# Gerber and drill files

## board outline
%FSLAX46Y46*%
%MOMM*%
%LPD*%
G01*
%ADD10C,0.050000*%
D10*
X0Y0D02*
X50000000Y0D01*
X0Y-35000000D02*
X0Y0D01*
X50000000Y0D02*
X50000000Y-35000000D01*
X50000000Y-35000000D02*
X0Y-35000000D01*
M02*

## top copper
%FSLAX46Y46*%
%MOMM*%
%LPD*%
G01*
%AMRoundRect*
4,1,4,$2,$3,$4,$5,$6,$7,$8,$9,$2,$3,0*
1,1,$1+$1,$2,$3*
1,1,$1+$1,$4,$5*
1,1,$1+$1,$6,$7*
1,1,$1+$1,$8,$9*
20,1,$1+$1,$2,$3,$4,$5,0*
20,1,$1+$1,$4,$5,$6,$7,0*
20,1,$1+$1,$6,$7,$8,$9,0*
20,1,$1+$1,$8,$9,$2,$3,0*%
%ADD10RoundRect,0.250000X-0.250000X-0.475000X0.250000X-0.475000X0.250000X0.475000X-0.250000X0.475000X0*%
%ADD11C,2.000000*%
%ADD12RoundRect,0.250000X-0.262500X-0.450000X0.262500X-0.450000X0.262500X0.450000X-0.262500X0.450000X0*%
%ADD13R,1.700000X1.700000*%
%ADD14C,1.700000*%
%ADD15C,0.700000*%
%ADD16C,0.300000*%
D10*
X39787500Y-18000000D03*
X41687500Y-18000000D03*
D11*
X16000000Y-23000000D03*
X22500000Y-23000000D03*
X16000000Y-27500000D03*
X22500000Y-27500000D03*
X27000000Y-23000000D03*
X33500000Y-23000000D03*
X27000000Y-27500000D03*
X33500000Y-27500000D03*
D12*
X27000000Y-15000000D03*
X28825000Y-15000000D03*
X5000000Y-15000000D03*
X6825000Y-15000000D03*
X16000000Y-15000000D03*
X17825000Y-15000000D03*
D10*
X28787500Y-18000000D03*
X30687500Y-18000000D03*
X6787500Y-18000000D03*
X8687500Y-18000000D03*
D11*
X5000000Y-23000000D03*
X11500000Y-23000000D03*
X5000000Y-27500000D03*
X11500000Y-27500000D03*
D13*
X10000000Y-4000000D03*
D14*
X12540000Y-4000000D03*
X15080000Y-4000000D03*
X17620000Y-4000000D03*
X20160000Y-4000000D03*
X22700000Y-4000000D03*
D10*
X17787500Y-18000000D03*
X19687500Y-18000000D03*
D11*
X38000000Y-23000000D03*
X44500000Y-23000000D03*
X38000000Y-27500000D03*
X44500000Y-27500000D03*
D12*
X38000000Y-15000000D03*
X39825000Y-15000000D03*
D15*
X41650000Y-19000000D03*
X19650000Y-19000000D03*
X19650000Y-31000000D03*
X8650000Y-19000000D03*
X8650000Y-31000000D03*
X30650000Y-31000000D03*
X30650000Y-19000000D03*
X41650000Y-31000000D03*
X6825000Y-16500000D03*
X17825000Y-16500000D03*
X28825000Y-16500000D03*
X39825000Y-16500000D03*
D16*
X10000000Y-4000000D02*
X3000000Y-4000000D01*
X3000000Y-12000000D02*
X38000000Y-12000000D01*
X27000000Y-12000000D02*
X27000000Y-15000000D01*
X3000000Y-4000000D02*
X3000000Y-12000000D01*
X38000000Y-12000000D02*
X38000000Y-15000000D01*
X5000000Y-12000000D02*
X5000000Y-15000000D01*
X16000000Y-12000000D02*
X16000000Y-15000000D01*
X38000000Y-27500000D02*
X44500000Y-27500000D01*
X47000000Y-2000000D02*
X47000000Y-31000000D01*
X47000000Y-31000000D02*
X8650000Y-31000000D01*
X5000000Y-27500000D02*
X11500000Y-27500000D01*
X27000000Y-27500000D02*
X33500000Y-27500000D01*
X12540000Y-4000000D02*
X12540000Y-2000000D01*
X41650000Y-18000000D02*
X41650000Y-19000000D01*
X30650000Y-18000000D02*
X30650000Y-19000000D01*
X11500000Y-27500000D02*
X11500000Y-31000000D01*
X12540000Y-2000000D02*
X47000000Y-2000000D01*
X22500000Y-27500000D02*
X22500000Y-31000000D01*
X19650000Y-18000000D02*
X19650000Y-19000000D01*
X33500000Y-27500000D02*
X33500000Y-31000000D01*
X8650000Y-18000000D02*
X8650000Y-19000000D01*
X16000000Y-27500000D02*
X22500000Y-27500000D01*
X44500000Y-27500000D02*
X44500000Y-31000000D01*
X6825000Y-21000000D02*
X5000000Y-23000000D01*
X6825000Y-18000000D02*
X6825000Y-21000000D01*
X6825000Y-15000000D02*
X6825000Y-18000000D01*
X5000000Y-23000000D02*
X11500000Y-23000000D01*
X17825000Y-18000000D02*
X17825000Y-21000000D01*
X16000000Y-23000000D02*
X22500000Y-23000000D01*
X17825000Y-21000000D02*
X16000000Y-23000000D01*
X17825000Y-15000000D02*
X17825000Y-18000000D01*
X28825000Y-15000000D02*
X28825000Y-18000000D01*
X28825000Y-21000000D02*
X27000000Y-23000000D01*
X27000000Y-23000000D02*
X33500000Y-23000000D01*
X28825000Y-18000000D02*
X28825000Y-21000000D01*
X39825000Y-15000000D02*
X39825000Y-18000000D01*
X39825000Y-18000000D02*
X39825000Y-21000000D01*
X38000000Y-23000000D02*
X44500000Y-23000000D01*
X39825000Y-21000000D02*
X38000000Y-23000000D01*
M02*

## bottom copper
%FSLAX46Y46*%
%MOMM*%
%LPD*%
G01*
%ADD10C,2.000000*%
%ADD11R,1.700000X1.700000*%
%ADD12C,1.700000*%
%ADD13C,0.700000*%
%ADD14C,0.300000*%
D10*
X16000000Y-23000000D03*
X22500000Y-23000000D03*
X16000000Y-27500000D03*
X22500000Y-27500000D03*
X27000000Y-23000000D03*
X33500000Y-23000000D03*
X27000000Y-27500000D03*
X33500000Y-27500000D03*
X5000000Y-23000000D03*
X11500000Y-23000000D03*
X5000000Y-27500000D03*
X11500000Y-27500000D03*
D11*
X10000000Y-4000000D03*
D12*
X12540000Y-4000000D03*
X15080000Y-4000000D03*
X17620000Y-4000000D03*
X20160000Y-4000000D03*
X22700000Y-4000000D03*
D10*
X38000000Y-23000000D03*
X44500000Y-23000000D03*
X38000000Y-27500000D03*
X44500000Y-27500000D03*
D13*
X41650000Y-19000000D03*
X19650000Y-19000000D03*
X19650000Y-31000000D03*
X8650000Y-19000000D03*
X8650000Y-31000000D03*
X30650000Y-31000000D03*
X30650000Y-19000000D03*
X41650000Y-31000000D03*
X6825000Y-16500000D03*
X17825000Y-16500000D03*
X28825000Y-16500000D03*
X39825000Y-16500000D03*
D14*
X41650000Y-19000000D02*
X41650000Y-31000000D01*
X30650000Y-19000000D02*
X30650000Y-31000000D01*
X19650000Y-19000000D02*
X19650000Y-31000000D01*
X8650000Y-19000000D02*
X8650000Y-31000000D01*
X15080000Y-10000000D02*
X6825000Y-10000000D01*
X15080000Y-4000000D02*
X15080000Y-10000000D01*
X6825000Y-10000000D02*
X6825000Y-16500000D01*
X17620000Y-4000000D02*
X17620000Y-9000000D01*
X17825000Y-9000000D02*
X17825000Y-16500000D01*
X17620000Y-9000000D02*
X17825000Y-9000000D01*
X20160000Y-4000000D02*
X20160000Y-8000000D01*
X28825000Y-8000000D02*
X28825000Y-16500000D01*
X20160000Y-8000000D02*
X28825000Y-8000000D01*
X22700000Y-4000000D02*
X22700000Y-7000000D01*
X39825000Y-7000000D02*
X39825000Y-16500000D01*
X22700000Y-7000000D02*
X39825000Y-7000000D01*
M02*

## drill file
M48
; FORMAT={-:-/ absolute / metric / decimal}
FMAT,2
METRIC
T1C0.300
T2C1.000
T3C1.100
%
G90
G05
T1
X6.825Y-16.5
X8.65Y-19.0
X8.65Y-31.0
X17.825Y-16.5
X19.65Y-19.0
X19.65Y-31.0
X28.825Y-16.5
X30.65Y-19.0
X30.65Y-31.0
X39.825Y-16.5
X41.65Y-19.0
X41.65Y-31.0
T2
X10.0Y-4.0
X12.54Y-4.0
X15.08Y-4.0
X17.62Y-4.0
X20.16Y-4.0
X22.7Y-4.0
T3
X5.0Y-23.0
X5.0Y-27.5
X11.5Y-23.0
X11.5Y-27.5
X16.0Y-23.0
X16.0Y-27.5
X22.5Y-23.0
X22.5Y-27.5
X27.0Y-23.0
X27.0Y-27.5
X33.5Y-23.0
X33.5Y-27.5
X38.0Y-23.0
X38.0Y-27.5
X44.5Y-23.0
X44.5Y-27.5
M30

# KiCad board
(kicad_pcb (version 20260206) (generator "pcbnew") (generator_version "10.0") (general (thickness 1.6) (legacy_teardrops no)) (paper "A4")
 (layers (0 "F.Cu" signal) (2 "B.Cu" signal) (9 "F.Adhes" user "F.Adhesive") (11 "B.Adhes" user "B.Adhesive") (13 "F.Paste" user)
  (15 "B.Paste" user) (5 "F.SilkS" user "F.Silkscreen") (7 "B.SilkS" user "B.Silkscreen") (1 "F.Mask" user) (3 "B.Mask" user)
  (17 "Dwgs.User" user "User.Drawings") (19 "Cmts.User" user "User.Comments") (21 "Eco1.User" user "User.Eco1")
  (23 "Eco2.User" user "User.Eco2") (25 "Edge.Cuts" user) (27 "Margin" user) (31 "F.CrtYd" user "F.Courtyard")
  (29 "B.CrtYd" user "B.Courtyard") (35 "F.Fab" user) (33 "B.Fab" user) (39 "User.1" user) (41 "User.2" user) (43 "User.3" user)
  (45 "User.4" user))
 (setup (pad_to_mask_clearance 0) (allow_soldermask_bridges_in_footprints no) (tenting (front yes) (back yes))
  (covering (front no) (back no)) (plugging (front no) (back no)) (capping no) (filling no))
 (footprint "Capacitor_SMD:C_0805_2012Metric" (layer "F.Cu") (at 40.7375 18)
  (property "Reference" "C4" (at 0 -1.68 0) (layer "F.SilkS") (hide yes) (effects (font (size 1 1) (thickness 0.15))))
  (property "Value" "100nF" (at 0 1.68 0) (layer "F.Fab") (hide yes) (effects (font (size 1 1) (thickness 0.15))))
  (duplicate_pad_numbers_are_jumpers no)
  (pad "1" smd roundrect (at -0.95 0) (size 1 1.45) (layers "F.Cu" "F.Mask" "F.Paste") (roundrect_rratio 0.25) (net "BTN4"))
  (pad "2" smd roundrect (at 0.95 0) (size 1 1.45) (layers "F.Cu" "F.Mask" "F.Paste") (roundrect_rratio 0.25) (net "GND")))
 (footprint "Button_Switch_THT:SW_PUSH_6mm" (layer "F.Cu") (at 16 23)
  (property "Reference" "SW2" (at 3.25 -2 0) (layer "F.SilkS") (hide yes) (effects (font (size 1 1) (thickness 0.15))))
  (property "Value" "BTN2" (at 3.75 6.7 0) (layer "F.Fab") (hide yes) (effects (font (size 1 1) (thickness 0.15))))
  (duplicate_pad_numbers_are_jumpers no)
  (pad "1" thru_hole circle (at 0 0 90) (size 2 2) (drill 1.1) (layers "*.Cu" "*.Mask") (remove_unused_layers no) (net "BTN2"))
  (pad "1" thru_hole circle (at 6.5 0 90) (size 2 2) (drill 1.1) (layers "*.Cu" "*.Mask") (remove_unused_layers no) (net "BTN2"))
  (pad "2" thru_hole circle (at 0 4.5 90) (size 2 2) (drill 1.1) (layers "*.Cu" "*.Mask") (remove_unused_layers no) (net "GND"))
  (pad "2" thru_hole circle (at 6.5 4.5 90) (size 2 2) (drill 1.1) (layers "*.Cu" "*.Mask") (remove_unused_layers no) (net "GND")))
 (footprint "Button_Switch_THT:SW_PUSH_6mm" (layer "F.Cu") (at 27 23)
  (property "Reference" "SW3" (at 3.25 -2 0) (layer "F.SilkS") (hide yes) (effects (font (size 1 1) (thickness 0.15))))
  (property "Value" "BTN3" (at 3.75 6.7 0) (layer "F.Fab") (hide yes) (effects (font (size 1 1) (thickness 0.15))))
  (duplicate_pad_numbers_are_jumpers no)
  (pad "1" thru_hole circle (at 0 0 90) (size 2 2) (drill 1.1) (layers "*.Cu" "*.Mask") (remove_unused_layers no) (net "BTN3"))
  (pad "1" thru_hole circle (at 6.5 0 90) (size 2 2) (drill 1.1) (layers "*.Cu" "*.Mask") (remove_unused_layers no) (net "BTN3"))
  (pad "2" thru_hole circle (at 0 4.5 90) (size 2 2) (drill 1.1) (layers "*.Cu" "*.Mask") (remove_unused_layers no) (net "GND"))
  (pad "2" thru_hole circle (at 6.5 4.5 90) (size 2 2) (drill 1.1) (layers "*.Cu" "*.Mask") (remove_unused_layers no) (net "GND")))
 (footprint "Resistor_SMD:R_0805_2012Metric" (layer "F.Cu") (at 27.9125 15)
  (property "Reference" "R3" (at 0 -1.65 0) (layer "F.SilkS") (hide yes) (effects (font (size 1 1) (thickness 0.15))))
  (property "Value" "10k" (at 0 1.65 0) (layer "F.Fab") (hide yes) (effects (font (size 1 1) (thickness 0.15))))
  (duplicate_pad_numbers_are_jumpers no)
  (pad "1" smd roundrect (at -0.9125 0) (size 1.025 1.4) (layers "F.Cu" "F.Mask" "F.Paste") (roundrect_rratio 0.243902) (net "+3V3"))
  (pad "2" smd roundrect (at 0.9125 0) (size 1.025 1.4) (layers "F.Cu" "F.Mask" "F.Paste") (roundrect_rratio 0.243902) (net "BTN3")))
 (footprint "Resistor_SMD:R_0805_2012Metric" (layer "F.Cu") (at 5.9125 15)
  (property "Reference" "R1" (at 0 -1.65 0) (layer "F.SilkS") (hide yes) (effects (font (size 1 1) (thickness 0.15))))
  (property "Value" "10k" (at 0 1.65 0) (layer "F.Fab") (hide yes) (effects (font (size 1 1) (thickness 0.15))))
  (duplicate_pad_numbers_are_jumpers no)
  (pad "1" smd roundrect (at -0.9125 0) (size 1.025 1.4) (layers "F.Cu" "F.Mask" "F.Paste") (roundrect_rratio 0.243902) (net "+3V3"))
  (pad "2" smd roundrect (at 0.9125 0) (size 1.025 1.4) (layers "F.Cu" "F.Mask" "F.Paste") (roundrect_rratio 0.243902) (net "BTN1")))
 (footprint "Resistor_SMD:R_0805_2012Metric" (layer "F.Cu") (at 16.9125 15)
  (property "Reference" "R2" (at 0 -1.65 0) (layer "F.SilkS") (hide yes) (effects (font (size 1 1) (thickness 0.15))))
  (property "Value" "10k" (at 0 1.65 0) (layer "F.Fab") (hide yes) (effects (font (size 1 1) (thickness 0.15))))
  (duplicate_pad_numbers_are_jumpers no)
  (pad "1" smd roundrect (at -0.9125 0) (size 1.025 1.4) (layers "F.Cu" "F.Mask" "F.Paste") (roundrect_rratio 0.243902) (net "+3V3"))
  (pad "2" smd roundrect (at 0.9125 0) (size 1.025 1.4) (layers "F.Cu" "F.Mask" "F.Paste") (roundrect_rratio 0.243902) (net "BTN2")))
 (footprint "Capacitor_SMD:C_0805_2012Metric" (layer "F.Cu") (at 29.7375 18)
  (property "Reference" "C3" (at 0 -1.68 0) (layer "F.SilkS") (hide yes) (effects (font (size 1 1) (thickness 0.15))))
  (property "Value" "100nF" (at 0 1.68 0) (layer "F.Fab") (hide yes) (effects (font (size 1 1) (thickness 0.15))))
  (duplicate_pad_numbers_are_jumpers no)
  (pad "1" smd roundrect (at -0.95 0) (size 1 1.45) (layers "F.Cu" "F.Mask" "F.Paste") (roundrect_rratio 0.25) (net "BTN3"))
  (pad "2" smd roundrect (at 0.95 0) (size 1 1.45) (layers "F.Cu" "F.Mask" "F.Paste") (roundrect_rratio 0.25) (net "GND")))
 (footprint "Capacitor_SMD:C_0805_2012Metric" (layer "F.Cu") (at 7.7375 18)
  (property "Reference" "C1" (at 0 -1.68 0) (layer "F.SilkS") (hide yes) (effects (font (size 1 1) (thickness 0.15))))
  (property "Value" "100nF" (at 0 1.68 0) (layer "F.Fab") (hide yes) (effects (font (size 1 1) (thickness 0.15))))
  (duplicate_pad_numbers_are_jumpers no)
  (pad "1" smd roundrect (at -0.95 0) (size 1 1.45) (layers "F.Cu" "F.Mask" "F.Paste") (roundrect_rratio 0.25) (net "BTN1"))
  (pad "2" smd roundrect (at 0.95 0) (size 1 1.45) (layers "F.Cu" "F.Mask" "F.Paste") (roundrect_rratio 0.25) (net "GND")))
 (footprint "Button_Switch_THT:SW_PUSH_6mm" (layer "F.Cu") (at 5 23)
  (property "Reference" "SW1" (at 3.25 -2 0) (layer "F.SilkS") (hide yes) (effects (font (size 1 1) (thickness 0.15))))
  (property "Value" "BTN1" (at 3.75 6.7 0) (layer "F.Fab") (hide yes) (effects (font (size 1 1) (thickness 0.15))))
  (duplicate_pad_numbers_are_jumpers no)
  (pad "1" thru_hole circle (at 0 0 90) (size 2 2) (drill 1.1) (layers "*.Cu" "*.Mask") (remove_unused_layers no) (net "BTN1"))
  (pad "1" thru_hole circle (at 6.5 0 90) (size 2 2) (drill 1.1) (layers "*.Cu" "*.Mask") (remove_unused_layers no) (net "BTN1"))
  (pad "2" thru_hole circle (at 0 4.5 90) (size 2 2) (drill 1.1) (layers "*.Cu" "*.Mask") (remove_unused_layers no) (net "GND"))
  (pad "2" thru_hole circle (at 6.5 4.5 90) (size 2 2) (drill 1.1) (layers "*.Cu" "*.Mask") (remove_unused_layers no) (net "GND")))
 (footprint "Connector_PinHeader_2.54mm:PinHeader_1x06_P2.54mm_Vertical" (layer "F.Cu") (at 10 4 90)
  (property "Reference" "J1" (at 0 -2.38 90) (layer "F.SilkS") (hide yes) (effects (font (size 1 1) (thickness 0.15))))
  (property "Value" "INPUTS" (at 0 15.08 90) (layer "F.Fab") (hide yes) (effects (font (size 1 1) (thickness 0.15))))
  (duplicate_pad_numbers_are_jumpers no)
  (pad "1" thru_hole rect (at 0 0 90) (size 1.7 1.7) (drill 1) (layers "*.Cu" "*.Mask") (remove_unused_layers no) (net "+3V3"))
  (pad "2" thru_hole circle (at 0 2.54 90) (size 1.7 1.7) (drill 1) (layers "*.Cu" "*.Mask") (remove_unused_layers no) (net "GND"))
  (pad "3" thru_hole circle (at 0 5.08 90) (size 1.7 1.7) (drill 1) (layers "*.Cu" "*.Mask") (remove_unused_layers no) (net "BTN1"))
  (pad "4" thru_hole circle (at 0 7.62 90) (size 1.7 1.7) (drill 1) (layers "*.Cu" "*.Mask") (remove_unused_layers no) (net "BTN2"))
  (pad "5" thru_hole circle (at 0 10.16 90) (size 1.7 1.7) (drill 1) (layers "*.Cu" "*.Mask") (remove_unused_layers no) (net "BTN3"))
  (pad "6" thru_hole circle (at 0 12.7 90) (size 1.7 1.7) (drill 1) (layers "*.Cu" "*.Mask") (remove_unused_layers no) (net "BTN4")))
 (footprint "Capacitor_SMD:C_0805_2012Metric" (layer "F.Cu") (at 18.7375 18)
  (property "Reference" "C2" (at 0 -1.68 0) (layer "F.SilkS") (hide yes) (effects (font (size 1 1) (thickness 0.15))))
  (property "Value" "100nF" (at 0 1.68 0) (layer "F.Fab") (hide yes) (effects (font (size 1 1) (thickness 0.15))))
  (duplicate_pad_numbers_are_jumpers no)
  (pad "1" smd roundrect (at -0.95 0) (size 1 1.45) (layers "F.Cu" "F.Mask" "F.Paste") (roundrect_rratio 0.25) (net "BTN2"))
  (pad "2" smd roundrect (at 0.95 0) (size 1 1.45) (layers "F.Cu" "F.Mask" "F.Paste") (roundrect_rratio 0.25) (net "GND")))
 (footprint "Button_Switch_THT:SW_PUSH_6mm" (layer "F.Cu") (at 38 23)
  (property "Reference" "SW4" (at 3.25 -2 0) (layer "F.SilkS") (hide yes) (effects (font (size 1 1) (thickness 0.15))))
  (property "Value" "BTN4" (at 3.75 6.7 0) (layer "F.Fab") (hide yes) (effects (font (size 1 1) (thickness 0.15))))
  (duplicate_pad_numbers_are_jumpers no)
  (pad "1" thru_hole circle (at 0 0 90) (size 2 2) (drill 1.1) (layers "*.Cu" "*.Mask") (remove_unused_layers no) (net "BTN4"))
  (pad "1" thru_hole circle (at 6.5 0 90) (size 2 2) (drill 1.1) (layers "*.Cu" "*.Mask") (remove_unused_layers no) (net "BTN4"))
  (pad "2" thru_hole circle (at 0 4.5 90) (size 2 2) (drill 1.1) (layers "*.Cu" "*.Mask") (remove_unused_layers no) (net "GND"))
  (pad "2" thru_hole circle (at 6.5 4.5 90) (size 2 2) (drill 1.1) (layers "*.Cu" "*.Mask") (remove_unused_layers no) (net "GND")))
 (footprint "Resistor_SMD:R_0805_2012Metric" (layer "F.Cu") (at 38.9125 15)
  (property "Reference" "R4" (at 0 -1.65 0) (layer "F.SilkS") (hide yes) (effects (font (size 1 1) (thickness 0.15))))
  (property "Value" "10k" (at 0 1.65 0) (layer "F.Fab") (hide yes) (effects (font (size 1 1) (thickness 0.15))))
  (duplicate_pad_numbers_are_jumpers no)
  (pad "1" smd roundrect (at -0.9125 0) (size 1.025 1.4) (layers "F.Cu" "F.Mask" "F.Paste") (roundrect_rratio 0.243902) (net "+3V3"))
  (pad "2" smd roundrect (at 0.9125 0) (size 1.025 1.4) (layers "F.Cu" "F.Mask" "F.Paste") (roundrect_rratio 0.243902) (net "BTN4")))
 (gr_line (start 0 0) (end 50 0) (stroke (width 0.05) (type default)) (layer "Edge.Cuts"))
 (gr_line (start 0 35) (end 0 0) (stroke (width 0.05) (type default)) (layer "Edge.Cuts"))
 (gr_line (start 50 0) (end 50 35) (stroke (width 0.05) (type default)) (layer "Edge.Cuts"))
 (gr_line (start 50 35) (end 0 35) (stroke (width 0.05) (type default)) (layer "Edge.Cuts"))
 (segment (start 10 4) (end 3 4) (width 0.3) (layer "F.Cu") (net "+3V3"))
 (segment (start 3 12) (end 38 12) (width 0.3) (layer "F.Cu") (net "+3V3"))
 (segment (start 27 12) (end 27 15) (width 0.3) (layer "F.Cu") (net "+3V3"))
 (segment (start 3 4) (end 3 12) (width 0.3) (layer "F.Cu") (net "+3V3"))
 (segment (start 38 12) (end 38 15) (width 0.3) (layer "F.Cu") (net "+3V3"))
 (segment (start 5 12) (end 5 15) (width 0.3) (layer "F.Cu") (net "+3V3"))
 (segment (start 16 12) (end 16 15) (width 0.3) (layer "F.Cu") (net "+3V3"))
 (segment (start 38 27.5) (end 44.5 27.5) (width 0.3) (layer "F.Cu") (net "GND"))
 (segment (start 47 2) (end 47 31) (width 0.3) (layer "F.Cu") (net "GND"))
 (segment (start 47 31) (end 8.65 31) (width 0.3) (layer "F.Cu") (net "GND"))
 (segment (start 5 27.5) (end 11.5 27.5) (width 0.3) (layer "F.Cu") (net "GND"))
 (segment (start 27 27.5) (end 33.5 27.5) (width 0.3) (layer "F.Cu") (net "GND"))
 (segment (start 12.54 4) (end 12.54 2) (width 0.3) (layer "F.Cu") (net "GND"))
 (segment (start 41.65 18) (end 41.65 19) (width 0.3) (layer "F.Cu") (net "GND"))
 (segment (start 30.65 18) (end 30.65 19) (width 0.3) (layer "F.Cu") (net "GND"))
 (segment (start 11.5 27.5) (end 11.5 31) (width 0.3) (layer "F.Cu") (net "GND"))
 (segment (start 12.54 2) (end 47 2) (width 0.3) (layer "F.Cu") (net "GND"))
 (segment (start 22.5 27.5) (end 22.5 31) (width 0.3) (layer "F.Cu") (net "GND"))
 (segment (start 19.65 18) (end 19.65 19) (width 0.3) (layer "F.Cu") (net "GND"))
 (segment (start 33.5 27.5) (end 33.5 31) (width 0.3) (layer "F.Cu") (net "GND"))
 (segment (start 8.65 18) (end 8.65 19) (width 0.3) (layer "F.Cu") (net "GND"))
 (segment (start 16 27.5) (end 22.5 27.5) (width 0.3) (layer "F.Cu") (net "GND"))
 (segment (start 44.5 27.5) (end 44.5 31) (width 0.3) (layer "F.Cu") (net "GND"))
 (via (at 41.65 19) (size 0.7) (drill 0.3) (layers "F.Cu" "B.Cu") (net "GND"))
 (via (at 19.65 19) (size 0.7) (drill 0.3) (layers "F.Cu" "B.Cu") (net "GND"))
 (via (at 19.65 31) (size 0.7) (drill 0.3) (layers "F.Cu" "B.Cu") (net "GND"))
 (via (at 8.65 19) (size 0.7) (drill 0.3) (layers "F.Cu" "B.Cu") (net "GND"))
 (via (at 8.65 31) (size 0.7) (drill 0.3) (layers "F.Cu" "B.Cu") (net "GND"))
 (via (at 30.65 31) (size 0.7) (drill 0.3) (layers "F.Cu" "B.Cu") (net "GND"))
 (via (at 30.65 19) (size 0.7) (drill 0.3) (layers "F.Cu" "B.Cu") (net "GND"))
 (via (at 41.65 31) (size 0.7) (drill 0.3) (layers "F.Cu" "B.Cu") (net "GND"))
 (segment (start 41.65 19) (end 41.65 31) (width 0.3) (layer "B.Cu") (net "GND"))
 (segment (start 30.65 19) (end 30.65 31) (width 0.3) (layer "B.Cu") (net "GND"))
 (segment (start 19.65 19) (end 19.65 31) (width 0.3) (layer "B.Cu") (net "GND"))
 (segment (start 8.65 19) (end 8.65 31) (width 0.3) (layer "B.Cu") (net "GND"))
 (segment (start 6.825 21) (end 5 23) (width 0.3) (layer "F.Cu") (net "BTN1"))
 (segment (start 6.825 18) (end 6.825 21) (width 0.3) (layer "F.Cu") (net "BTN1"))
 (segment (start 6.825 15) (end 6.825 18) (width 0.3) (layer "F.Cu") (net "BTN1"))
 (segment (start 5 23) (end 11.5 23) (width 0.3) (layer "F.Cu") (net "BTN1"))
 (via (at 6.825 16.5) (size 0.7) (drill 0.3) (layers "F.Cu" "B.Cu") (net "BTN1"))
 (segment (start 15.08 10) (end 6.825 10) (width 0.3) (layer "B.Cu") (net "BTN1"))
 (segment (start 15.08 4) (end 15.08 10) (width 0.3) (layer "B.Cu") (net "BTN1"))
 (segment (start 6.825 10) (end 6.825 16.5) (width 0.3) (layer "B.Cu") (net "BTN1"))
 (segment (start 17.825 18) (end 17.825 21) (width 0.3) (layer "F.Cu") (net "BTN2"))
 (segment (start 16 23) (end 22.5 23) (width 0.3) (layer "F.Cu") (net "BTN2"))
 (segment (start 17.825 21) (end 16 23) (width 0.3) (layer "F.Cu") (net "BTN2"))
 (segment (start 17.825 15) (end 17.825 18) (width 0.3) (layer "F.Cu") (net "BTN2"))
 (via (at 17.825 16.5) (size 0.7) (drill 0.3) (layers "F.Cu" "B.Cu") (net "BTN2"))
 (segment (start 17.62 4) (end 17.62 9) (width 0.3) (layer "B.Cu") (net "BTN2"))
 (segment (start 17.825 9) (end 17.825 16.5) (width 0.3) (layer "B.Cu") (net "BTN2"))
 (segment (start 17.62 9) (end 17.825 9) (width 0.3) (layer "B.Cu") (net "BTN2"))
 (segment (start 28.825 15) (end 28.825 18) (width 0.3) (layer "F.Cu") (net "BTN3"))
 (segment (start 28.825 21) (end 27 23) (width 0.3) (layer "F.Cu") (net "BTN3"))
 (segment (start 27 23) (end 33.5 23) (width 0.3) (layer "F.Cu") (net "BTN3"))
 (segment (start 28.825 18) (end 28.825 21) (width 0.3) (layer "F.Cu") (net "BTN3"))
 (via (at 28.825 16.5) (size 0.7) (drill 0.3) (layers "F.Cu" "B.Cu") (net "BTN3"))
 (segment (start 20.16 4) (end 20.16 8) (width 0.3) (layer "B.Cu") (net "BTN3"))
 (segment (start 28.825 8) (end 28.825 16.5) (width 0.3) (layer "B.Cu") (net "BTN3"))
 (segment (start 20.16 8) (end 28.825 8) (width 0.3) (layer "B.Cu") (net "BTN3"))
 (segment (start 39.825 15) (end 39.825 18) (width 0.3) (layer "F.Cu") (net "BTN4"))
 (segment (start 39.825 18) (end 39.825 21) (width 0.3) (layer "F.Cu") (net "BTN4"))
 (segment (start 38 23) (end 44.5 23) (width 0.3) (layer "F.Cu") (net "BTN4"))
 (segment (start 39.825 21) (end 38 23) (width 0.3) (layer "F.Cu") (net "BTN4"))
 (via (at 39.825 16.5) (size 0.7) (drill 0.3) (layers "F.Cu" "B.Cu") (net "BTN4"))
 (segment (start 22.7 4) (end 22.7 7) (width 0.3) (layer "B.Cu") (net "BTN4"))
 (segment (start 39.825 7) (end 39.825 16.5) (width 0.3) (layer "B.Cu") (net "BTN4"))
 (segment (start 22.7 7) (end 39.825 7) (width 0.3) (layer "B.Cu") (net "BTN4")))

